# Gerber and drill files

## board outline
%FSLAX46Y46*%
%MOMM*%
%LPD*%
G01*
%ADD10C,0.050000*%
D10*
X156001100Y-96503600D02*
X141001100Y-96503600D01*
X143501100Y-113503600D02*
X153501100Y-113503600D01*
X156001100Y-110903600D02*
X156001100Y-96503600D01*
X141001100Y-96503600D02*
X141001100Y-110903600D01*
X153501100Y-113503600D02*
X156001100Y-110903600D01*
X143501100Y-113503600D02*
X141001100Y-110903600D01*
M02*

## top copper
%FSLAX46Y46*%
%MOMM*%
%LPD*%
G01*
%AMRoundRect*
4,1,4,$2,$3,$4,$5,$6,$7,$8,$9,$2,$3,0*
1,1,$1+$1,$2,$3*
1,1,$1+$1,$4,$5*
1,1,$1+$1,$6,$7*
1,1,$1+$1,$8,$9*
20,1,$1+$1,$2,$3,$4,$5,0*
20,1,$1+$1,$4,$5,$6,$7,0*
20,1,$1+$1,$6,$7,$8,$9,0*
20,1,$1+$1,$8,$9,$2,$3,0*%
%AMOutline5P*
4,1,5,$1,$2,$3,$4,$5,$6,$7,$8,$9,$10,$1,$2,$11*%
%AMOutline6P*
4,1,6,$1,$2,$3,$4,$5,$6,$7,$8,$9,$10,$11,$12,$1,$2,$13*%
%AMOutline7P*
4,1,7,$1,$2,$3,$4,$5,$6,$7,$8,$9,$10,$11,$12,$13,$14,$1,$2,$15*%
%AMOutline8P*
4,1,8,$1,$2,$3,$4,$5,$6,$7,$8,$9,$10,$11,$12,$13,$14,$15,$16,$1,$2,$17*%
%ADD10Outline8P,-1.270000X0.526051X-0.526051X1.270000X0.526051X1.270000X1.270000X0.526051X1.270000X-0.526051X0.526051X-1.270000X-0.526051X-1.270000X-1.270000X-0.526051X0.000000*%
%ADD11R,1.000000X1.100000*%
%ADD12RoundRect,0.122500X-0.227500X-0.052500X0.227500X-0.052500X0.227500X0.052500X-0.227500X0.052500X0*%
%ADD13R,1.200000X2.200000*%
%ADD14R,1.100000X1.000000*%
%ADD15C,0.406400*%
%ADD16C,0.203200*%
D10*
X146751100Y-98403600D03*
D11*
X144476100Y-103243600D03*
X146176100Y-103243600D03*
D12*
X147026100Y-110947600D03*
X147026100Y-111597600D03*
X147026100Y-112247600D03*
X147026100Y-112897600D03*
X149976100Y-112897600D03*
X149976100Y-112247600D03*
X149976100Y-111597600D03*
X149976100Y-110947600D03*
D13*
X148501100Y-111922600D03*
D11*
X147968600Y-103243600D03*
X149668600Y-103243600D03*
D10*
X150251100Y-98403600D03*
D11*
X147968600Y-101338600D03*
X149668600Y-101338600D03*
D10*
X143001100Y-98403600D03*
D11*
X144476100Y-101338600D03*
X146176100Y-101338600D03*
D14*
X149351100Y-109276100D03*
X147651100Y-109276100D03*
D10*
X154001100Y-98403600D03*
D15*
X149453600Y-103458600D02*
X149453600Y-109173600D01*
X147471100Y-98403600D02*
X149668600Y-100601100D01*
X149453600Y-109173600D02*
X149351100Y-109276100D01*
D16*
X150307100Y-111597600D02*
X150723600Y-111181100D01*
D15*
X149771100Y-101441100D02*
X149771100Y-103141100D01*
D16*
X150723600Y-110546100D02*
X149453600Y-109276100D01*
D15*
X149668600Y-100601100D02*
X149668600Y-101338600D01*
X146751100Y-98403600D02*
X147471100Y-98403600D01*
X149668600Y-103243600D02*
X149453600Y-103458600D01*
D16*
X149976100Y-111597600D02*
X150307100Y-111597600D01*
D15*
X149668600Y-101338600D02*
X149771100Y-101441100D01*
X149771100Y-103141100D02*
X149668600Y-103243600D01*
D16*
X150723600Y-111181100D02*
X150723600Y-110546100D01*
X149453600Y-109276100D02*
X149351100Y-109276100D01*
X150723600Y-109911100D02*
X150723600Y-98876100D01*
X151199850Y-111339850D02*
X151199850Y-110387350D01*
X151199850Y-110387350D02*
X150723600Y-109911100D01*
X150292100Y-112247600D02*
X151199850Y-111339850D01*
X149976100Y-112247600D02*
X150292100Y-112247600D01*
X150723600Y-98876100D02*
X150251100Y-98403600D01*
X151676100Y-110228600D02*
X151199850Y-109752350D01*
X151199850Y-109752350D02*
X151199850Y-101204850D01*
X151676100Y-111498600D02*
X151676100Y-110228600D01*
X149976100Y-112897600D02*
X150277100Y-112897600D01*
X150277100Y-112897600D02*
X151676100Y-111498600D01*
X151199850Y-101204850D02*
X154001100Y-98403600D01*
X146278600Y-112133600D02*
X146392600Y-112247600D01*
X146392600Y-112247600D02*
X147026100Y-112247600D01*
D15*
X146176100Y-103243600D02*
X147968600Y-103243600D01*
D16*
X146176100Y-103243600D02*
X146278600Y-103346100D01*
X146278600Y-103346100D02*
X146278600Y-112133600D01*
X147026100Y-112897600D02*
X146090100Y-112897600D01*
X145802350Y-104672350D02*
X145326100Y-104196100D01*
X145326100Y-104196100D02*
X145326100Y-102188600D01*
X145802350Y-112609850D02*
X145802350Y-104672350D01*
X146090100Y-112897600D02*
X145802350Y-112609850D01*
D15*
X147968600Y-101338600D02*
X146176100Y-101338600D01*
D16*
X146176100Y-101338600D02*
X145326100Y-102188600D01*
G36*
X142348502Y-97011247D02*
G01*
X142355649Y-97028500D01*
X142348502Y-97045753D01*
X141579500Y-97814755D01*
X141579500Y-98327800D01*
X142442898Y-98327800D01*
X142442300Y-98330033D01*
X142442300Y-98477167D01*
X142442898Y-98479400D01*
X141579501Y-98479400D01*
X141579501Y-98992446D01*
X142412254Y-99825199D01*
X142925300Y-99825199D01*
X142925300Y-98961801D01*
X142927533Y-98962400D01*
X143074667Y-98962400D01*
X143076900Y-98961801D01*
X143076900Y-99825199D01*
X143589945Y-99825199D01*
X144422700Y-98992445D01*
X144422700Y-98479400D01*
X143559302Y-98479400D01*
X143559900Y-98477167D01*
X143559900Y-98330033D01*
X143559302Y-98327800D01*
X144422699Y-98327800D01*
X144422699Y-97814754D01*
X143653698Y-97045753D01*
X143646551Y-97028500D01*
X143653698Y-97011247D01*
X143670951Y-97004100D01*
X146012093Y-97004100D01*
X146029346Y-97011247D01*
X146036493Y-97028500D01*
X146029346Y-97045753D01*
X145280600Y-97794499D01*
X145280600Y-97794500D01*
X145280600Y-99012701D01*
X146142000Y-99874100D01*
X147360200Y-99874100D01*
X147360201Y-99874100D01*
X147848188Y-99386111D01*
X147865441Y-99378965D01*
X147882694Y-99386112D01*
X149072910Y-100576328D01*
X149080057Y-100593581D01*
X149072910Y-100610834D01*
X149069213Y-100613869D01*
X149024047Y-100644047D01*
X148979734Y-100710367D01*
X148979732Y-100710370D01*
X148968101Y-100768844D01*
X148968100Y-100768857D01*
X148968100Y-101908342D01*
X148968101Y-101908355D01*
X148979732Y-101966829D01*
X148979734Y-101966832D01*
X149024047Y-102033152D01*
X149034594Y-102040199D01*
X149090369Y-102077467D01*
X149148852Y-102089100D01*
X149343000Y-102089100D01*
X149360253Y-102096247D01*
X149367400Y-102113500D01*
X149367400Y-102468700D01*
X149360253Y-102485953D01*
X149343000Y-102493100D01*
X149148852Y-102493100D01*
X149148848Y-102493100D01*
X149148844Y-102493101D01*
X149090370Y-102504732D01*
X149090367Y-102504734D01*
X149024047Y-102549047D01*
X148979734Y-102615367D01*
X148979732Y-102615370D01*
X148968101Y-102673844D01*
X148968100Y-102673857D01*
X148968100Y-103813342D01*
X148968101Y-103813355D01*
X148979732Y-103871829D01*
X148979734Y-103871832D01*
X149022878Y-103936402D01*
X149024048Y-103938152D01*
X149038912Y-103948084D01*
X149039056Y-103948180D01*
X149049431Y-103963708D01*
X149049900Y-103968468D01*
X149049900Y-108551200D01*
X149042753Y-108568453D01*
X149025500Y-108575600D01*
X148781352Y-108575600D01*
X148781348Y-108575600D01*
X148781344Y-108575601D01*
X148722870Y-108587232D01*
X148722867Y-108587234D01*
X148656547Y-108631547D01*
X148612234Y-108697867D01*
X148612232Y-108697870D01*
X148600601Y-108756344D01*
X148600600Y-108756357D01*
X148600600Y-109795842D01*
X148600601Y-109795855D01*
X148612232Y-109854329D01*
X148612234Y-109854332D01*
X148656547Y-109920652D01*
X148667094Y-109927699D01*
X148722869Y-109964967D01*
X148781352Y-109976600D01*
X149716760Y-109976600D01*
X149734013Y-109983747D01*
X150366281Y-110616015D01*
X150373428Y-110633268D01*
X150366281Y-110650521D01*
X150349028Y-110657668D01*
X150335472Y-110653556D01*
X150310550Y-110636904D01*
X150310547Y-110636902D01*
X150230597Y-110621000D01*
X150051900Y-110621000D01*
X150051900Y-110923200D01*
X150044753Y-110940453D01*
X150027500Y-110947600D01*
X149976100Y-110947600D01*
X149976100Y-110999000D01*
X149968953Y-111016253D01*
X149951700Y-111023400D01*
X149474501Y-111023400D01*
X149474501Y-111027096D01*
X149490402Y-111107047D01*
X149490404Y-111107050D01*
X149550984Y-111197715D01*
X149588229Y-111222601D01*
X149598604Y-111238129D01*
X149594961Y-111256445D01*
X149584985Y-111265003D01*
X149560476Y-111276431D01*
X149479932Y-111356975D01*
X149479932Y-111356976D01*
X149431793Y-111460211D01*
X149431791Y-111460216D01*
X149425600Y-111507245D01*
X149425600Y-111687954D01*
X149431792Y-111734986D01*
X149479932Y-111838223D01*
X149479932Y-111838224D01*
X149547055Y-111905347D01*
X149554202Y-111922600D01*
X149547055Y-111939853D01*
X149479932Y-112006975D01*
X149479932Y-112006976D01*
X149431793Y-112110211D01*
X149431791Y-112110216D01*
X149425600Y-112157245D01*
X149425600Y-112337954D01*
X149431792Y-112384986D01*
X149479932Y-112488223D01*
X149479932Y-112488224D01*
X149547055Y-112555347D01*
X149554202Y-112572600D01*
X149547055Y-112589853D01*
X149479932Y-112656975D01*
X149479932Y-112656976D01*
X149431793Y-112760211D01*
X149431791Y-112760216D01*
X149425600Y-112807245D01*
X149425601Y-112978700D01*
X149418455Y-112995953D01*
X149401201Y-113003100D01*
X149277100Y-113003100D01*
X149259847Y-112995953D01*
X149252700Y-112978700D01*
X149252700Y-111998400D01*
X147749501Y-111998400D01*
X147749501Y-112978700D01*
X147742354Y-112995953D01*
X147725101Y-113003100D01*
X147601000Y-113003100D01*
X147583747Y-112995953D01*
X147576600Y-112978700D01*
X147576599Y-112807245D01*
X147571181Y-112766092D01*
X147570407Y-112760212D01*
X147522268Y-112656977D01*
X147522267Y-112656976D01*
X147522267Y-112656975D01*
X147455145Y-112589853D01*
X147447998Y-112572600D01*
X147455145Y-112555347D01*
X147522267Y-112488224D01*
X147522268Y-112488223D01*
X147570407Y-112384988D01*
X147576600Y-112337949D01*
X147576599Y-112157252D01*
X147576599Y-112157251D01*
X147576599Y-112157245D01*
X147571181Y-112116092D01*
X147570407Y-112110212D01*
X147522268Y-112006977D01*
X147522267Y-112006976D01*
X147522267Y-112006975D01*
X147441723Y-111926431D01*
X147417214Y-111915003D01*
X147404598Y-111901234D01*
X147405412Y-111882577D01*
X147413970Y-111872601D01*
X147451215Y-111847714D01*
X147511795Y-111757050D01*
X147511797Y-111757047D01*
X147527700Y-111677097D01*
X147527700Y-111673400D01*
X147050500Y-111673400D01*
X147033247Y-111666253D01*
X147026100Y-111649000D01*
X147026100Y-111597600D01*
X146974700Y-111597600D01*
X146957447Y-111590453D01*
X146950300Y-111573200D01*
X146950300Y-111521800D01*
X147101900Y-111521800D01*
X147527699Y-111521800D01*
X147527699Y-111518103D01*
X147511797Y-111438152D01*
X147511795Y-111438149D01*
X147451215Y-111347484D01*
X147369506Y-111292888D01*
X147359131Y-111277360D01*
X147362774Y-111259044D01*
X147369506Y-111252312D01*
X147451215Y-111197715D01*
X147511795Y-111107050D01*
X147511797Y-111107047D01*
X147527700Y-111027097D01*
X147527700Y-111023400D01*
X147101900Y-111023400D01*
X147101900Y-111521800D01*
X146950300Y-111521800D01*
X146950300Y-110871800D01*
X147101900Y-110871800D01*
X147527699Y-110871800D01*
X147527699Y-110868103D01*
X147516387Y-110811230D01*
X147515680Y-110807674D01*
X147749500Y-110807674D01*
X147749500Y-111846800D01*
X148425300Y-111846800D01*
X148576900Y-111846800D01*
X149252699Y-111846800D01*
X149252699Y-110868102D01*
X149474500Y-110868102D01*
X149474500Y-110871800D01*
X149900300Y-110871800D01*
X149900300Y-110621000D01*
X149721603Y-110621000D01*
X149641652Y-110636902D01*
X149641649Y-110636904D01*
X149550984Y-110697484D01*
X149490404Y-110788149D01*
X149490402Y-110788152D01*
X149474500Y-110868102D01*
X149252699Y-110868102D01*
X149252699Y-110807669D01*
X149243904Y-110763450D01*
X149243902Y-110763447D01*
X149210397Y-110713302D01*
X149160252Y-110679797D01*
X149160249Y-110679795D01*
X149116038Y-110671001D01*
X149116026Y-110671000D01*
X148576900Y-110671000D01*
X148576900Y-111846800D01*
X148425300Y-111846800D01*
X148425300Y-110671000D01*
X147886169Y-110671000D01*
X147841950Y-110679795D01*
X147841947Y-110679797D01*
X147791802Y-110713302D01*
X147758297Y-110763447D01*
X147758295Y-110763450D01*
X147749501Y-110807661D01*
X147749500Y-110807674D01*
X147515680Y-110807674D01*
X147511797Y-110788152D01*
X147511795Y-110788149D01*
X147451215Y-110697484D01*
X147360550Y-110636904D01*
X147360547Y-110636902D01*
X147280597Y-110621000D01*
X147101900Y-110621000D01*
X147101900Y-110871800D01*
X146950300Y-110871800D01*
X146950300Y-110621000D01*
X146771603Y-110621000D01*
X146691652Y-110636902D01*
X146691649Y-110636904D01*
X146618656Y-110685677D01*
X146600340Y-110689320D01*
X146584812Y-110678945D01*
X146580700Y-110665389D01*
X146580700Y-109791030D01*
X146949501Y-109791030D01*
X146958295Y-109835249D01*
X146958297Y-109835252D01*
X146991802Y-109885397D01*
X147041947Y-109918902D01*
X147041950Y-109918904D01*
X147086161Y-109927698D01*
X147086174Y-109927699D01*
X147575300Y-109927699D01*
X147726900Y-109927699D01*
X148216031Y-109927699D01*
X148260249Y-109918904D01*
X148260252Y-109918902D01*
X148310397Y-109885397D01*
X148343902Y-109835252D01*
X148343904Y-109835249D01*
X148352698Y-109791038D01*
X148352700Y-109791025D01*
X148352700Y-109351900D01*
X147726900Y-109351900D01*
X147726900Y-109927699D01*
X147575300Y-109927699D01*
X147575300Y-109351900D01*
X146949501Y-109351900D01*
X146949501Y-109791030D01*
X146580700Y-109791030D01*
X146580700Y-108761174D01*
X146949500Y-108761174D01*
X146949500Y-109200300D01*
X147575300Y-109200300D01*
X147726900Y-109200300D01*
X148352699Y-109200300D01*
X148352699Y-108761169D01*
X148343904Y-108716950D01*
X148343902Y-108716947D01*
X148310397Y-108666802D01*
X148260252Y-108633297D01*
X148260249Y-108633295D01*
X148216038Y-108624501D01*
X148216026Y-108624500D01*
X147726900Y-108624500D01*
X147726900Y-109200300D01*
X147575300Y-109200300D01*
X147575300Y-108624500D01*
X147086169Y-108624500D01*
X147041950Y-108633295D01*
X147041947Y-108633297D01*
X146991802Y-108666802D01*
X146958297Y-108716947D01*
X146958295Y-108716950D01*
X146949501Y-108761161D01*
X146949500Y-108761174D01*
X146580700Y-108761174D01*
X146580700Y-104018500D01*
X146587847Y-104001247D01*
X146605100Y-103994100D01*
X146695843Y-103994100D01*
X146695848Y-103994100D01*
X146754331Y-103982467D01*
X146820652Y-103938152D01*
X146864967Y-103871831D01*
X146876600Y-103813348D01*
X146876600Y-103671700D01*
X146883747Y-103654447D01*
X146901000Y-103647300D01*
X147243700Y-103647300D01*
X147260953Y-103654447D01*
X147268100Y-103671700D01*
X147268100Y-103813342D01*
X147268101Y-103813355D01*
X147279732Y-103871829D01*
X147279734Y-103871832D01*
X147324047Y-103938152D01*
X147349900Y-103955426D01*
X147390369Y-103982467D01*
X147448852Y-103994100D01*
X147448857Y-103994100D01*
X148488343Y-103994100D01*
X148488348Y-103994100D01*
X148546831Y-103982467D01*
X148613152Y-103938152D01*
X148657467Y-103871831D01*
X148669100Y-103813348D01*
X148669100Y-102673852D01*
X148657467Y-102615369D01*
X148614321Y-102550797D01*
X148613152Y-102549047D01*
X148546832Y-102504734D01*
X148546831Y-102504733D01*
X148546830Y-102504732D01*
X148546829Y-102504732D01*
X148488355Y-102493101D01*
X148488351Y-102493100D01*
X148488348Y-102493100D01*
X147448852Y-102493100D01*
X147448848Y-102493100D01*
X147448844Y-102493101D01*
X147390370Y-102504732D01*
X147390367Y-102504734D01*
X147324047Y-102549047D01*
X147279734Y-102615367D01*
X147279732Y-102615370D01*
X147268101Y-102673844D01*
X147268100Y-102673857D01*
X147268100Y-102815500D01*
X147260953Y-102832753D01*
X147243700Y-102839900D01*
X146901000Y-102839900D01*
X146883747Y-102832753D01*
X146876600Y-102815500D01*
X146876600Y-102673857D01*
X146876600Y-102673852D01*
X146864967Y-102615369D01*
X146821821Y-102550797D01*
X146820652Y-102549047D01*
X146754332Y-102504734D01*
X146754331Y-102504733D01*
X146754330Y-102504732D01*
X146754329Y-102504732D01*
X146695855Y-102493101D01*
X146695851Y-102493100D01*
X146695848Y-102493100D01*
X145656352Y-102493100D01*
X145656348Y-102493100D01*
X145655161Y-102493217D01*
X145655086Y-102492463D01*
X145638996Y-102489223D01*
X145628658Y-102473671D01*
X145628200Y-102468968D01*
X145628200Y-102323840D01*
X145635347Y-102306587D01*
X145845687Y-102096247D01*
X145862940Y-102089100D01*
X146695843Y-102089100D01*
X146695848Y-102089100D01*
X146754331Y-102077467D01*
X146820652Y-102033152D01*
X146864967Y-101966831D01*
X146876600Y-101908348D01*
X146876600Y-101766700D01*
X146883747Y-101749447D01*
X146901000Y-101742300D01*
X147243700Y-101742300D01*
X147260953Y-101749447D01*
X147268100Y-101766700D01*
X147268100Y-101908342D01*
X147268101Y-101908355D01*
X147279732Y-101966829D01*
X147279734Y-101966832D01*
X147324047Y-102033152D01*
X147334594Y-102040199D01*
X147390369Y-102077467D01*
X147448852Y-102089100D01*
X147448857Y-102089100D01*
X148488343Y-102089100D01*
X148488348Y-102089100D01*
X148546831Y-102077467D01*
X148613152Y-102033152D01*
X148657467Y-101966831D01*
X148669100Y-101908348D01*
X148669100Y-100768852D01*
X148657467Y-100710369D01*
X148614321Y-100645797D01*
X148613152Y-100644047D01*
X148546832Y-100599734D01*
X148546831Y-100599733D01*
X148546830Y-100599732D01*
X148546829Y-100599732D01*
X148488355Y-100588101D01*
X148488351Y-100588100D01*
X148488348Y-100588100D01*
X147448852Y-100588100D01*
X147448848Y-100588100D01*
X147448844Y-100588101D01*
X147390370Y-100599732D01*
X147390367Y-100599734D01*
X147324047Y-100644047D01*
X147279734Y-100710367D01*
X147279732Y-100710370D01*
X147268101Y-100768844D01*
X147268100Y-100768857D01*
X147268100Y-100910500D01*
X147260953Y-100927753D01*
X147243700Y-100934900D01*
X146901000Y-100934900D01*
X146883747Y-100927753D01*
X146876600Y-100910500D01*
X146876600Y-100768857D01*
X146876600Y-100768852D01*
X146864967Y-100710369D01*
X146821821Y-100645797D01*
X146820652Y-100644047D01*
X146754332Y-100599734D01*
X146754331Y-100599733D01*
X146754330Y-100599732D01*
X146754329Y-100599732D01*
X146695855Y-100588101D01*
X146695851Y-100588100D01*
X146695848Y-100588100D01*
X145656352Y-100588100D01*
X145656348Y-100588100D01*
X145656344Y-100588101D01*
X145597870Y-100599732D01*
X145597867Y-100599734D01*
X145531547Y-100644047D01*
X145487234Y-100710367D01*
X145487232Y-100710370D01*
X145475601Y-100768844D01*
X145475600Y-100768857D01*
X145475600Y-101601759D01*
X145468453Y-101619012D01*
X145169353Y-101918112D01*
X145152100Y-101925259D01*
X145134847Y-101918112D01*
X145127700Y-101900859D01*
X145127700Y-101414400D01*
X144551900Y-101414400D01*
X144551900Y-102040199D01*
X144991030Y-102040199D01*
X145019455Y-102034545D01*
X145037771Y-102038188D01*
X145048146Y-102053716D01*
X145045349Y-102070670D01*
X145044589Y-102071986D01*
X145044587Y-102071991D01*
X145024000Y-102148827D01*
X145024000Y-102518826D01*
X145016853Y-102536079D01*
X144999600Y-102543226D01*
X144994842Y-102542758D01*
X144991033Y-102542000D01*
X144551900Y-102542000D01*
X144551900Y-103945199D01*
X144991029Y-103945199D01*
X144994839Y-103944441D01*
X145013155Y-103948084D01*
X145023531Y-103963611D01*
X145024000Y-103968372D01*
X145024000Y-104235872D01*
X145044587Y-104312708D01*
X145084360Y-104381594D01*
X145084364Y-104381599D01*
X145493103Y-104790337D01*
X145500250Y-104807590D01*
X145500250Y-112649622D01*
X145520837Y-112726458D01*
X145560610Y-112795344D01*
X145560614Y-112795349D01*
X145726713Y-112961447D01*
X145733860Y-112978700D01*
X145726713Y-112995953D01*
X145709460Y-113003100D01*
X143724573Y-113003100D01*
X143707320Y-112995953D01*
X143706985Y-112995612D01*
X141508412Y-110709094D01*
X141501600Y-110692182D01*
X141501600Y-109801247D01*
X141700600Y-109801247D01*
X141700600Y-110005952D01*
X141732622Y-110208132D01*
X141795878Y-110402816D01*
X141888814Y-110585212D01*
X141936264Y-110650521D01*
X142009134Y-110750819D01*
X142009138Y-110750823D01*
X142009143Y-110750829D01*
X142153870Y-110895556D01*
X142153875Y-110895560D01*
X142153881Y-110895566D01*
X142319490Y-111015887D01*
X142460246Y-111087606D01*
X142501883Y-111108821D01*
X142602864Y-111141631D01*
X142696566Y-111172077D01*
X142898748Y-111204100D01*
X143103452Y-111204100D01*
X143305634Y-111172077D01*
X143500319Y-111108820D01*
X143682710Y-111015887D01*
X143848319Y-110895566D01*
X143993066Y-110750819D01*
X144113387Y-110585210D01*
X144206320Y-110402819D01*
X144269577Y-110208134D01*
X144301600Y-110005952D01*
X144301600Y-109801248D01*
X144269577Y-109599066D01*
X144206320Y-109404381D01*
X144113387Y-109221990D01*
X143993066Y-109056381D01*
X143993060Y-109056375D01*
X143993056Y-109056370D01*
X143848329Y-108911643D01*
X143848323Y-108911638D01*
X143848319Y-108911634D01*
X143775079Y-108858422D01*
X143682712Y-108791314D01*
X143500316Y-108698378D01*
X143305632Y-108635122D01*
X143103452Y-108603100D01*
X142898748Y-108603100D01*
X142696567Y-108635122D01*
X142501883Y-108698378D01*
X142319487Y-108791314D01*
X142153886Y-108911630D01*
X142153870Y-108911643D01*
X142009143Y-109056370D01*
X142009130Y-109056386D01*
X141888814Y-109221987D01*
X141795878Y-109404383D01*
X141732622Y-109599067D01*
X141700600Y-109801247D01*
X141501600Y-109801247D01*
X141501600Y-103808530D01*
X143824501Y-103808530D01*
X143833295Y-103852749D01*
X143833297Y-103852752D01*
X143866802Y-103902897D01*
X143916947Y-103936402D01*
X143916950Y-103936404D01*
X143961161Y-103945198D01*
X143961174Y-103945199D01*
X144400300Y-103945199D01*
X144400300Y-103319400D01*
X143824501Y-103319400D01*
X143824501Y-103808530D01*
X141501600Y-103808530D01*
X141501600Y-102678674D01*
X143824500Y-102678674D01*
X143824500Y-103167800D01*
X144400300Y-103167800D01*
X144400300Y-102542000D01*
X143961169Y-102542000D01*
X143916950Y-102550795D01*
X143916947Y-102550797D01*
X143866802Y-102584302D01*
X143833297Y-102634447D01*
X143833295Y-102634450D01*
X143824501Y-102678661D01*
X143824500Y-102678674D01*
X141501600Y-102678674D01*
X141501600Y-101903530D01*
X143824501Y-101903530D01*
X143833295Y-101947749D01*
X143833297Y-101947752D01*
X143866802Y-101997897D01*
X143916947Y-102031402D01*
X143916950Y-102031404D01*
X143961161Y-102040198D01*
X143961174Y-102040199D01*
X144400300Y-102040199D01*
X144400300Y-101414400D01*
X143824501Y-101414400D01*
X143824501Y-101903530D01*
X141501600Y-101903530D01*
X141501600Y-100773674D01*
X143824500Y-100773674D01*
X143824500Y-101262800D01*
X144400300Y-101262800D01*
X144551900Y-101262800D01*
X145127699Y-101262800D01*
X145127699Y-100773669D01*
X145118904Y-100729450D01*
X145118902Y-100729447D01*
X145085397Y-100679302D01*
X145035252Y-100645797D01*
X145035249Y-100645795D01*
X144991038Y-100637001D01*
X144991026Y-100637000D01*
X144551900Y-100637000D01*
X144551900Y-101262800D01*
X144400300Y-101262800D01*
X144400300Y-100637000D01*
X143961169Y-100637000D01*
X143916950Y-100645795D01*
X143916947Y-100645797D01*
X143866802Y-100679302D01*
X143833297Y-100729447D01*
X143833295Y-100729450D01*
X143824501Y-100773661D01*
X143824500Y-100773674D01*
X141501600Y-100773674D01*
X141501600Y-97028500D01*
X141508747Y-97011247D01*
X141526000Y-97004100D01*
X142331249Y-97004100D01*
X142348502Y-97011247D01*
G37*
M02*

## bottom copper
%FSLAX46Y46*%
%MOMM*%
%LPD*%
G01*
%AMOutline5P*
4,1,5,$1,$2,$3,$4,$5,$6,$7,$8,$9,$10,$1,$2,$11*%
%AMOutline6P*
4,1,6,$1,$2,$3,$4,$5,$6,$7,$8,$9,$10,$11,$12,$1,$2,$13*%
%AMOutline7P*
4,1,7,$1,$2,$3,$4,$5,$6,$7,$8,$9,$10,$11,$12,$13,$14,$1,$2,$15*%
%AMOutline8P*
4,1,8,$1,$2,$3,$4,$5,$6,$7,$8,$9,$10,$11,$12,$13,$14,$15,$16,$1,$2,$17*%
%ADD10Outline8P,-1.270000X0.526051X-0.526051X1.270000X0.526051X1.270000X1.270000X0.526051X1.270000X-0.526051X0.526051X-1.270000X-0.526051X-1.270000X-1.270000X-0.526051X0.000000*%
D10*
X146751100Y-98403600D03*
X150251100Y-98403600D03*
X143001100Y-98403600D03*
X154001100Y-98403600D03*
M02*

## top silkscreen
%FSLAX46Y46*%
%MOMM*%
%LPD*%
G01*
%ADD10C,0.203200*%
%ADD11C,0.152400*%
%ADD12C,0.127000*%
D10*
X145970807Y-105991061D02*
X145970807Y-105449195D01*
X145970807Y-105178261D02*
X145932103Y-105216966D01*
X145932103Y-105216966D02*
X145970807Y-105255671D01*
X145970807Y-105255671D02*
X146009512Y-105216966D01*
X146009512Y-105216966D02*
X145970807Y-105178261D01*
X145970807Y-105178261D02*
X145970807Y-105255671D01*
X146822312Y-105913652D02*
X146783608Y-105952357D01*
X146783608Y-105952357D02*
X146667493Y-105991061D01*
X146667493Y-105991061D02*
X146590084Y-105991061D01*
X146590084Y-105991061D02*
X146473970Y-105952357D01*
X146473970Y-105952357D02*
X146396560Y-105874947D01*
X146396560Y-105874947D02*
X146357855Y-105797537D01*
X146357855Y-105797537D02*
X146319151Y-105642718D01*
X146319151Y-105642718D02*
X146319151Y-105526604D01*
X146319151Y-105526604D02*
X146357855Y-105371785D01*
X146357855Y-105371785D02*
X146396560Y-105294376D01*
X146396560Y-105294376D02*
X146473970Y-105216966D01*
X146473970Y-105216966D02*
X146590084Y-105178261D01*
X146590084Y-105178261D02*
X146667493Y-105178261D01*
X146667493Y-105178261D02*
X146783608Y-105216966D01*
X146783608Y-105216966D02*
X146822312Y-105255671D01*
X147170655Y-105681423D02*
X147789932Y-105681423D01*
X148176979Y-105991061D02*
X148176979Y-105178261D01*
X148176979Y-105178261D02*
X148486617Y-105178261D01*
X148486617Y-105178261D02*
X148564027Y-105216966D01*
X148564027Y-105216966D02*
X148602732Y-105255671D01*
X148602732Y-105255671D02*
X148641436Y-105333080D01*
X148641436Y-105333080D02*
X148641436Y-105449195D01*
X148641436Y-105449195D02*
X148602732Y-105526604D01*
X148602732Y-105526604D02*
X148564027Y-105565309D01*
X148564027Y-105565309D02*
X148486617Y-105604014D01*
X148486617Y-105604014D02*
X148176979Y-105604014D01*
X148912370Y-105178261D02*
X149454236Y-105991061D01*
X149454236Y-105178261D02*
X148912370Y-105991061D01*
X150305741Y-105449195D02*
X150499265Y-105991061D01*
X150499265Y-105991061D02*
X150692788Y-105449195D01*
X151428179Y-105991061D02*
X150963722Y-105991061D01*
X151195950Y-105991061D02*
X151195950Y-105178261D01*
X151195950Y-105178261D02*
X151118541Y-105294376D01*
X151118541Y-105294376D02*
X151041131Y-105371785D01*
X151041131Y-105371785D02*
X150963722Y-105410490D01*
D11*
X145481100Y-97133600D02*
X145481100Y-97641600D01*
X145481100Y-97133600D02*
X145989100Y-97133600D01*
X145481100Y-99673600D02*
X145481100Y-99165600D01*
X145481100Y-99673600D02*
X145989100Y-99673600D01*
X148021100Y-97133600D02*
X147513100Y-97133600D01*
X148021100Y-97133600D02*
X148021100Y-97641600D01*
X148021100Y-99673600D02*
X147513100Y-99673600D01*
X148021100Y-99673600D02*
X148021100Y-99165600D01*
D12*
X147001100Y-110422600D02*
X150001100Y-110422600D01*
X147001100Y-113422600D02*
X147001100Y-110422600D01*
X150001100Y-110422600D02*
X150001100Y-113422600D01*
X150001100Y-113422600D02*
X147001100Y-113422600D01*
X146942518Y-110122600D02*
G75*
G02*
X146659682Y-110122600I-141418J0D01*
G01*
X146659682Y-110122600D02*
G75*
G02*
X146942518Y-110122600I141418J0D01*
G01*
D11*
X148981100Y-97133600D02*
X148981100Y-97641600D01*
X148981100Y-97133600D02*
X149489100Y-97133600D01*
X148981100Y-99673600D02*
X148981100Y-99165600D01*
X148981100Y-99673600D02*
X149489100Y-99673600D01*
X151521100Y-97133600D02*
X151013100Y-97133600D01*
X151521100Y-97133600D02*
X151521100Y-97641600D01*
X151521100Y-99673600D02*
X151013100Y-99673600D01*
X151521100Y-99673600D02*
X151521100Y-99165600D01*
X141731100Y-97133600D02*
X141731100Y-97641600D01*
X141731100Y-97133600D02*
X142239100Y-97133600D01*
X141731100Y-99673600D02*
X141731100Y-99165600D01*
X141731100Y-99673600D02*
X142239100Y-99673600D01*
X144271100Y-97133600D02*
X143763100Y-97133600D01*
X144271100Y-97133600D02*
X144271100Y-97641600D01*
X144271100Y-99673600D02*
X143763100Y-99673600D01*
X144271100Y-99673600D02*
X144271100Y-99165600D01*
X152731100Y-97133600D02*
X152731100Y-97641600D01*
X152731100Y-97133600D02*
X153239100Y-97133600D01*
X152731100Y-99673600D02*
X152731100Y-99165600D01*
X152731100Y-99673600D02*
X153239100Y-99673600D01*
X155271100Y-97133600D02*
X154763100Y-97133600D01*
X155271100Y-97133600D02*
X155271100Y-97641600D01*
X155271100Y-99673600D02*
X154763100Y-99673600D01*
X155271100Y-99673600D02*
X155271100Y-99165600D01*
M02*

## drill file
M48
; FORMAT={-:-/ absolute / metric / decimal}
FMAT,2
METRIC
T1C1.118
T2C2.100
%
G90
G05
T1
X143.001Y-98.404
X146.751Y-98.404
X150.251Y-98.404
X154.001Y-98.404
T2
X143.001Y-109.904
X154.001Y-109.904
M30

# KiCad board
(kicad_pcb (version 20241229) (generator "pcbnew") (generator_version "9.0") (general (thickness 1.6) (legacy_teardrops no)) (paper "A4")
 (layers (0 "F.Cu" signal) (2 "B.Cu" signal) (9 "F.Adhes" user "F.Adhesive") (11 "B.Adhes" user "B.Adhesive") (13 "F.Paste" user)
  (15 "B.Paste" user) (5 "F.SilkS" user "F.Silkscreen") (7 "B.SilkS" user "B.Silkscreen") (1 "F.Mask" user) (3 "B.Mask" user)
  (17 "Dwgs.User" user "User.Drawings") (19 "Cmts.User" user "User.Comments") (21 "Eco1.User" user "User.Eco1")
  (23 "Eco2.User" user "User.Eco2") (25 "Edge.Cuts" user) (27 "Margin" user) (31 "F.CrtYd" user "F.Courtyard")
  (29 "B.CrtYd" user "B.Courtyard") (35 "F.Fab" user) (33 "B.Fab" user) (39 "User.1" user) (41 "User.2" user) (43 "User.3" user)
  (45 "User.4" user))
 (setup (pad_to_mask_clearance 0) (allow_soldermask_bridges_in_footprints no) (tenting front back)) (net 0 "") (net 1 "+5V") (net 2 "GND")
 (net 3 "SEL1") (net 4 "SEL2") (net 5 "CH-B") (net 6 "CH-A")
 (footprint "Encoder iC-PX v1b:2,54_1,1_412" (layer "F.Cu") (at 146.7511 98.4036)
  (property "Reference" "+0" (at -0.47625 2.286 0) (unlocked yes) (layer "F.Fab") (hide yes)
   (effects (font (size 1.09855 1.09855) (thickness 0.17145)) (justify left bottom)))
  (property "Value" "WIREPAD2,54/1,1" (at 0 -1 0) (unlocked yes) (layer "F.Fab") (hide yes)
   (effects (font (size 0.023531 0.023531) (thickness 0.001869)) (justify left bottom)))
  (fp_line (start -1.27 -1.27) (end -1.27 -0.762) (stroke (width 0.1524) (type solid)) (layer "F.SilkS"))
  (fp_line (start -1.27 -1.27) (end -0.762 -1.27) (stroke (width 0.1524) (type solid)) (layer "F.SilkS"))
  (fp_line (start -1.27 1.27) (end -1.27 0.762) (stroke (width 0.1524) (type solid)) (layer "F.SilkS"))
  (fp_line (start -1.27 1.27) (end -0.762 1.27) (stroke (width 0.1524) (type solid)) (layer "F.SilkS"))
  (fp_line (start 1.27 -1.27) (end 0.762 -1.27) (stroke (width 0.1524) (type solid)) (layer "F.SilkS"))
  (fp_line (start 1.27 -1.27) (end 1.27 -0.762) (stroke (width 0.1524) (type solid)) (layer "F.SilkS"))
  (fp_line (start 1.27 1.27) (end 0.762 1.27) (stroke (width 0.1524) (type solid)) (layer "F.SilkS"))
  (fp_line (start 1.27 1.27) (end 1.27 0.762) (stroke (width 0.1524) (type solid)) (layer "F.SilkS"))
  (pad "1" thru_hole roundrect (at 0 0) (size 2.54 2.54) (drill 1.1176) (layers "*.Cu" "*.Mask") (remove_unused_layers no)
   (roundrect_rratio 0.25) (chamfer_ratio 0.2928932188) (chamfer top_left top_right bottom_left bottom_right) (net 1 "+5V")
   (solder_mask_margin 0.075) (thermal_bridge_angle 0)))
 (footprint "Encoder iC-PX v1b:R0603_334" (layer "F.Cu") (at 145.3261 103.2436)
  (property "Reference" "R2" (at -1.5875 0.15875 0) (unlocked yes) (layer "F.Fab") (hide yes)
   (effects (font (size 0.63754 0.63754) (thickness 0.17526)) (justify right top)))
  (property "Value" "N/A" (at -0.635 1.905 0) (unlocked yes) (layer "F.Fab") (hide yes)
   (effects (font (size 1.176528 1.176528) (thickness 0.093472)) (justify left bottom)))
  (pad "1" smd rect (at -0.85 0) (size 1 1.1) (layers "F.Cu" "F.Mask" "F.Paste") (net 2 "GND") (solder_mask_margin 0.075)
   (solder_paste_margin 0) (thermal_bridge_angle 0))
  (pad "2" smd rect (at 0.85 0) (size 1 1.1) (layers "F.Cu" "F.Mask" "F.Paste") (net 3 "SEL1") (solder_mask_margin 0.075)
   (solder_paste_margin 0) (thermal_bridge_angle 0)))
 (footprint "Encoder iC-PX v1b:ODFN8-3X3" (layer "F.Cu") (at 148.5011 111.9226)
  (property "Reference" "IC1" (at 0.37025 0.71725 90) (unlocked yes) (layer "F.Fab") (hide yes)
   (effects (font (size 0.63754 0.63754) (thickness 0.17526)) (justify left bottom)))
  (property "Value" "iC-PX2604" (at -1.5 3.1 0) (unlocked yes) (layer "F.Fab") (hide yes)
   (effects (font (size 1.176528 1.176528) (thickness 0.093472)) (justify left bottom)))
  (fp_line (start -1.5 -1.5) (end 1.5 -1.5) (stroke (width 0.127) (type solid)) (layer "F.SilkS"))
  (fp_line (start -1.5 1.5) (end -1.5 -1.5) (stroke (width 0.127) (type solid)) (layer "F.SilkS"))
  (fp_line (start 1.5 -1.5) (end 1.5 1.5) (stroke (width 0.127) (type solid)) (layer "F.SilkS"))
  (fp_line (start 1.5 1.5) (end -1.5 1.5) (stroke (width 0.127) (type solid)) (layer "F.SilkS"))
  (fp_circle (center -1.7 -1.8) (end -1.558582 -1.8) (stroke (width 0.127) (type solid)) (fill no) (layer "F.SilkS"))
  (pad "1" smd roundrect (at -1.475 -0.975) (size 0.7 0.35) (layers "F.Cu" "F.Mask" "F.Paste") (roundrect_rratio 0.35) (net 2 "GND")
   (solder_mask_margin 0.075) (solder_paste_margin 0) (thermal_bridge_angle 0))
  (pad "2" smd roundrect (at -1.475 -0.325) (size 0.7 0.35) (layers "F.Cu" "F.Mask" "F.Paste") (roundrect_rratio 0.35) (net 2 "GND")
   (solder_mask_margin 0.075) (solder_paste_margin 0) (thermal_bridge_angle 0))
  (pad "3" smd roundrect (at -1.475 0.325) (size 0.7 0.35) (layers "F.Cu" "F.Mask" "F.Paste") (roundrect_rratio 0.35) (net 3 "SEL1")
   (solder_mask_margin 0.075) (solder_paste_margin 0) (thermal_bridge_angle 0))
  (pad "4" smd roundrect (at -1.475 0.975) (size 0.7 0.35) (layers "F.Cu" "F.Mask" "F.Paste") (roundrect_rratio 0.35) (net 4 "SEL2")
   (solder_mask_margin 0.075) (solder_paste_margin 0) (thermal_bridge_angle 0))
  (pad "5" smd roundrect (at 1.475 0.975) (size 0.7 0.35) (layers "F.Cu" "F.Mask" "F.Paste") (roundrect_rratio 0.35) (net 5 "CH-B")
   (solder_mask_margin 0.075) (solder_paste_margin 0) (thermal_bridge_angle 0))
  (pad "6" smd roundrect (at 1.475 0.325) (size 0.7 0.35) (layers "F.Cu" "F.Mask" "F.Paste") (roundrect_rratio 0.35) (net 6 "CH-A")
   (solder_mask_margin 0.075) (solder_paste_margin 0) (thermal_bridge_angle 0))
  (pad "7" smd roundrect (at 1.475 -0.325) (size 0.7 0.35) (layers "F.Cu" "F.Mask" "F.Paste") (roundrect_rratio 0.35) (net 1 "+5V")
   (solder_mask_margin 0.075) (solder_paste_margin 0) (thermal_bridge_angle 0))
  (pad "8" smd roundrect (at 1.475 -0.975) (size 0.7 0.35) (layers "F.Cu" "F.Mask" "F.Paste") (roundrect_rratio 0.35) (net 2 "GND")
   (solder_mask_margin 0.075) (solder_paste_margin 0) (thermal_bridge_angle 0))
  (pad "BP" smd rect (at 0 0) (size 1.2 2.2) (layers "F.Cu" "F.Mask") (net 2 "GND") (solder_mask_margin 0.075) (solder_paste_margin 0)
   (thermal_bridge_angle 0)))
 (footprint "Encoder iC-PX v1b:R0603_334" (layer "F.Cu") (at 148.8186 103.2436)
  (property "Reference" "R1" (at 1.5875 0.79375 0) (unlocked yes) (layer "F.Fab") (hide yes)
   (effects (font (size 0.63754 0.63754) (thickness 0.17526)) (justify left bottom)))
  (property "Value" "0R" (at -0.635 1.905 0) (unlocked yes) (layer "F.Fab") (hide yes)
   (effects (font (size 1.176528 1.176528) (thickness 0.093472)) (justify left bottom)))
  (pad "1" smd rect (at -0.85 0) (size 1 1.1) (layers "F.Cu" "F.Mask" "F.Paste") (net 3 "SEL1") (solder_mask_margin 0.075)
   (solder_paste_margin 0) (thermal_bridge_angle 0))
  (pad "2" smd rect (at 0.85 0) (size 1 1.1) (layers "F.Cu" "F.Mask" "F.Paste") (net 1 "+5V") (solder_mask_margin 0.075)
   (solder_paste_margin 0) (thermal_bridge_angle 0)))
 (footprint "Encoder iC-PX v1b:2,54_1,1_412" (layer "F.Cu") (at 150.2511 98.4036)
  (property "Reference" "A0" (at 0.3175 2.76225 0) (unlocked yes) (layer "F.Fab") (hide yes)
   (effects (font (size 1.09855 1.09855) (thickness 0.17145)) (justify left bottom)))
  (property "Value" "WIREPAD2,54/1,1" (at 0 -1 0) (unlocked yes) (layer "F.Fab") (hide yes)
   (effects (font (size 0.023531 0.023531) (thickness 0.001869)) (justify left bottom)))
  (fp_line (start -1.27 -1.27) (end -1.27 -0.762) (stroke (width 0.1524) (type solid)) (layer "F.SilkS"))
  (fp_line (start -1.27 -1.27) (end -0.762 -1.27) (stroke (width 0.1524) (type solid)) (layer "F.SilkS"))
  (fp_line (start -1.27 1.27) (end -1.27 0.762) (stroke (width 0.1524) (type solid)) (layer "F.SilkS"))
  (fp_line (start -1.27 1.27) (end -0.762 1.27) (stroke (width 0.1524) (type solid)) (layer "F.SilkS"))
  (fp_line (start 1.27 -1.27) (end 0.762 -1.27) (stroke (width 0.1524) (type solid)) (layer "F.SilkS"))
  (fp_line (start 1.27 -1.27) (end 1.27 -0.762) (stroke (width 0.1524) (type solid)) (layer "F.SilkS"))
  (fp_line (start 1.27 1.27) (end 0.762 1.27) (stroke (width 0.1524) (type solid)) (layer "F.SilkS"))
  (fp_line (start 1.27 1.27) (end 1.27 0.762) (stroke (width 0.1524) (type solid)) (layer "F.SilkS"))
  (pad "1" thru_hole roundrect (at 0 0) (size 2.54 2.54) (drill 1.1176) (layers "*.Cu" "*.Mask") (remove_unused_layers no)
   (roundrect_rratio 0.25) (chamfer_ratio 0.2928932188) (chamfer top_left top_right bottom_left bottom_right) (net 6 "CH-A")
   (solder_mask_margin 0.075) (thermal_bridge_angle 0)))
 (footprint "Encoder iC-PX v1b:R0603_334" (layer "F.Cu") (at 148.8186 101.3386)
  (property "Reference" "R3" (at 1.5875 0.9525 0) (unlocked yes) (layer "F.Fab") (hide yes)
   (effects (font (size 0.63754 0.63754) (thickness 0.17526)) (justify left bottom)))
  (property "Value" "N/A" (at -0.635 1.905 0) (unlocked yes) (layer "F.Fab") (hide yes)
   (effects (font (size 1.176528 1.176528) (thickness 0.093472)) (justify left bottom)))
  (pad "1" smd rect (at -0.85 0) (size 1 1.1) (layers "F.Cu" "F.Mask" "F.Paste") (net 4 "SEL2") (solder_mask_margin 0.075)
   (solder_paste_margin 0) (thermal_bridge_angle 0))
  (pad "2" smd rect (at 0.85 0) (size 1 1.1) (layers "F.Cu" "F.Mask" "F.Paste") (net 1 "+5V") (solder_mask_margin 0.075)
   (solder_paste_margin 0) (thermal_bridge_angle 0)))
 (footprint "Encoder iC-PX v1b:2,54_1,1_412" (layer "F.Cu") (at 143.0011 98.4036)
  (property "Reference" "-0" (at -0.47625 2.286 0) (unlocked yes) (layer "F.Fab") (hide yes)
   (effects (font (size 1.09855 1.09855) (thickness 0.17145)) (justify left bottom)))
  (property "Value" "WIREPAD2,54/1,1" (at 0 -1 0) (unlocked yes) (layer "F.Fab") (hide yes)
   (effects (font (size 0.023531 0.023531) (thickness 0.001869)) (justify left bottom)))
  (fp_line (start -1.27 -1.27) (end -1.27 -0.762) (stroke (width 0.1524) (type solid)) (layer "F.SilkS"))
  (fp_line (start -1.27 -1.27) (end -0.762 -1.27) (stroke (width 0.1524) (type solid)) (layer "F.SilkS"))
  (fp_line (start -1.27 1.27) (end -1.27 0.762) (stroke (width 0.1524) (type solid)) (layer "F.SilkS"))
  (fp_line (start -1.27 1.27) (end -0.762 1.27) (stroke (width 0.1524) (type solid)) (layer "F.SilkS"))
  (fp_line (start 1.27 -1.27) (end 0.762 -1.27) (stroke (width 0.1524) (type solid)) (layer "F.SilkS"))
  (fp_line (start 1.27 -1.27) (end 1.27 -0.762) (stroke (width 0.1524) (type solid)) (layer "F.SilkS"))
  (fp_line (start 1.27 1.27) (end 0.762 1.27) (stroke (width 0.1524) (type solid)) (layer "F.SilkS"))
  (fp_line (start 1.27 1.27) (end 1.27 0.762) (stroke (width 0.1524) (type solid)) (layer "F.SilkS"))
  (pad "1" thru_hole roundrect (at 0 0) (size 2.54 2.54) (drill 1.1176) (layers "*.Cu" "*.Mask") (remove_unused_layers no)
   (roundrect_rratio 0.25) (chamfer_ratio 0.2928932188) (chamfer top_left top_right bottom_left bottom_right) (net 2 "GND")
   (solder_mask_margin 0.075) (thermal_bridge_angle 0)))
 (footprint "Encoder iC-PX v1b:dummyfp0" (layer "F.Cu") (at 143.0011 109.9036)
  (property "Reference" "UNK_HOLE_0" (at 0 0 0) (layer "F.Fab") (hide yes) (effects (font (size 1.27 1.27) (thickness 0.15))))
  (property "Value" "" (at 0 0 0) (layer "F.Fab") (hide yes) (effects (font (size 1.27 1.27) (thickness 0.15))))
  (pad "" np_thru_hole circle (at 0 0) (size 2.1 2.1) (drill 2.1) (layers "*.Cu" "*.Mask")))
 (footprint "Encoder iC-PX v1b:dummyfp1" (layer "F.Cu") (at 154.0011 109.9036)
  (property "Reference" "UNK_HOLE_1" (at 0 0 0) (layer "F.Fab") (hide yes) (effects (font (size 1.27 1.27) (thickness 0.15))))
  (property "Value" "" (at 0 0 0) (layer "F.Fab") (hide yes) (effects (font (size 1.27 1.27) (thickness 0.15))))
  (pad "" np_thru_hole circle (at 0 0) (size 2.1 2.1) (drill 2.1) (layers "*.Cu" "*.Mask")))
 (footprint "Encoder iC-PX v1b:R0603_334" (layer "F.Cu") (at 145.3261 101.3386)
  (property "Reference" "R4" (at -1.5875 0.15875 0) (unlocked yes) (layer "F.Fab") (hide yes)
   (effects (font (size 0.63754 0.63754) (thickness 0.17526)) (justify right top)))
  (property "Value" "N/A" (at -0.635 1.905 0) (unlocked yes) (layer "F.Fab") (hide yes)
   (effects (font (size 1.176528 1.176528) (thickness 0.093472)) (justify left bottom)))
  (pad "1" smd rect (at -0.85 0) (size 1 1.1) (layers "F.Cu" "F.Mask" "F.Paste") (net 2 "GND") (solder_mask_margin 0.075)
   (solder_paste_margin 0) (thermal_bridge_angle 0))
  (pad "2" smd rect (at 0.85 0) (size 1 1.1) (layers "F.Cu" "F.Mask" "F.Paste") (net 4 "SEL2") (solder_mask_margin 0.075)
   (solder_paste_margin 0) (thermal_bridge_angle 0)))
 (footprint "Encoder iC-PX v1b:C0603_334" (layer "F.Cu") (at 148.5011 109.2761 180)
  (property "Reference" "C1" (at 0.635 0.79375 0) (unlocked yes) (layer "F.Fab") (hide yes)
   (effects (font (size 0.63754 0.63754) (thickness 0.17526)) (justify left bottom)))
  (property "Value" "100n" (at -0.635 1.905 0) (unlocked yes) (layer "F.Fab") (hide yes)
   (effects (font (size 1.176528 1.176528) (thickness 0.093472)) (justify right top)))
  (pad "1" smd rect (at -0.85 0 180) (size 1.1 1) (layers "F.Cu" "F.Mask" "F.Paste") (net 1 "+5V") (solder_mask_margin 0.075)
   (solder_paste_margin 0) (thermal_bridge_angle 0))
  (pad "2" smd rect (at 0.85 0 180) (size 1.1 1) (layers "F.Cu" "F.Mask" "F.Paste") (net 2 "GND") (solder_mask_margin 0.075)
   (solder_paste_margin 0) (thermal_bridge_angle 0)))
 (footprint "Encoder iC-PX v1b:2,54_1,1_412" (layer "F.Cu") (at 154.0011 98.4036)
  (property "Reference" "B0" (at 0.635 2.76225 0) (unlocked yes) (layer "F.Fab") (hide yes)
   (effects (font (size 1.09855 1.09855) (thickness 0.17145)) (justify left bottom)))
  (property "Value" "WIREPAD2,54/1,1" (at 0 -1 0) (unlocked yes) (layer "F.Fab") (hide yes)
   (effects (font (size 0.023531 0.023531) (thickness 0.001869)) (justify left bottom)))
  (fp_line (start -1.27 -1.27) (end -1.27 -0.762) (stroke (width 0.1524) (type solid)) (layer "F.SilkS"))
  (fp_line (start -1.27 -1.27) (end -0.762 -1.27) (stroke (width 0.1524) (type solid)) (layer "F.SilkS"))
  (fp_line (start -1.27 1.27) (end -1.27 0.762) (stroke (width 0.1524) (type solid)) (layer "F.SilkS"))
  (fp_line (start -1.27 1.27) (end -0.762 1.27) (stroke (width 0.1524) (type solid)) (layer "F.SilkS"))
  (fp_line (start 1.27 -1.27) (end 0.762 -1.27) (stroke (width 0.1524) (type solid)) (layer "F.SilkS"))
  (fp_line (start 1.27 -1.27) (end 1.27 -0.762) (stroke (width 0.1524) (type solid)) (layer "F.SilkS"))
  (fp_line (start 1.27 1.27) (end 0.762 1.27) (stroke (width 0.1524) (type solid)) (layer "F.SilkS"))
  (fp_line (start 1.27 1.27) (end 1.27 0.762) (stroke (width 0.1524) (type solid)) (layer "F.SilkS"))
  (pad "1" thru_hole roundrect (at 0 0) (size 2.54 2.54) (drill 1.1176) (layers "*.Cu" "*.Mask") (remove_unused_layers no)
   (roundrect_rratio 0.25) (chamfer_ratio 0.2928932188) (chamfer top_left top_right bottom_left bottom_right) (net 5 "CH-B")
   (solder_mask_margin 0.075) (thermal_bridge_angle 0)))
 (gr_line (start 156.0011 96.5036) (end 141.0011 96.5036) (stroke (width 0.05) (type solid)) (layer "Edge.Cuts"))
 (gr_line (start 143.5011 113.5036) (end 153.5011 113.5036) (stroke (width 0.05) (type solid)) (layer "Edge.Cuts"))
 (gr_line (start 156.0011 110.9036) (end 156.0011 96.5036) (stroke (width 0.05) (type solid)) (layer "Edge.Cuts"))
 (gr_line (start 141.0011 96.5036) (end 141.0011 110.9036) (stroke (width 0.05) (type solid)) (layer "Edge.Cuts"))
 (gr_line (start 153.5011 113.5036) (end 156.0011 110.9036) (stroke (width 0.05) (type solid)) (layer "Edge.Cuts"))
 (gr_line (start 143.5011 113.5036) (end 141.0011 110.9036) (stroke (width 0.05) (type solid)) (layer "Edge.Cuts"))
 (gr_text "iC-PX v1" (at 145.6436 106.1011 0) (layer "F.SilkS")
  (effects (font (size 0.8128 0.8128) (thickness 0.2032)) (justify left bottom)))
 (segment (start 149.4536 103.4586) (end 149.4536 109.1736) (width 0.4064) (layer "F.Cu") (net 1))
 (segment (start 147.4711 98.4036) (end 149.6686 100.6011) (width 0.4064) (layer "F.Cu") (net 1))
 (segment (start 149.4536 109.1736) (end 149.3511 109.2761) (width 0.4064) (layer "F.Cu") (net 1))
 (segment (start 150.3071 111.5976) (end 150.7236 111.1811) (width 0.2032) (layer "F.Cu") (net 1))
 (segment (start 149.7711 101.4411) (end 149.7711 103.1411) (width 0.4064) (layer "F.Cu") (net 1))
 (segment (start 150.7236 110.5461) (end 149.4536 109.2761) (width 0.2032) (layer "F.Cu") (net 1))
 (segment (start 149.6686 100.6011) (end 149.6686 101.3386) (width 0.4064) (layer "F.Cu") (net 1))
 (segment (start 146.7511 98.4036) (end 147.4711 98.4036) (width 0.4064) (layer "F.Cu") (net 1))
 (segment (start 149.6686 103.2436) (end 149.4536 103.4586) (width 0.4064) (layer "F.Cu") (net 1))
 (segment (start 149.9761 111.5976) (end 150.3071 111.5976) (width 0.2032) (layer "F.Cu") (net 1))
 (segment (start 149.6686 101.3386) (end 149.7711 101.4411) (width 0.4064) (layer "F.Cu") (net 1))
 (segment (start 149.7711 103.1411) (end 149.6686 103.2436) (width 0.4064) (layer "F.Cu") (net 1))
 (segment (start 150.7236 111.1811) (end 150.7236 110.5461) (width 0.2032) (layer "F.Cu") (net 1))
 (segment (start 149.4536 109.2761) (end 149.3511 109.2761) (width 0.2032) (layer "F.Cu") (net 1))
 (segment (start 150.7236 109.9111) (end 150.7236 98.8761) (width 0.2032) (layer "F.Cu") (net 6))
 (segment (start 151.19985 111.33985) (end 151.19985 110.38735) (width 0.2032) (layer "F.Cu") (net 6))
 (segment (start 151.19985 110.38735) (end 150.7236 109.9111) (width 0.2032) (layer "F.Cu") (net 6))
 (segment (start 150.2921 112.2476) (end 151.19985 111.33985) (width 0.2032) (layer "F.Cu") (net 6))
 (segment (start 149.9761 112.2476) (end 150.2921 112.2476) (width 0.2032) (layer "F.Cu") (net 6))
 (segment (start 150.7236 98.8761) (end 150.2511 98.4036) (width 0.2032) (layer "F.Cu") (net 6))
 (segment (start 151.6761 110.2286) (end 151.19985 109.75235) (width 0.2032) (layer "F.Cu") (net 5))
 (segment (start 151.19985 109.75235) (end 151.19985 101.20485) (width 0.2032) (layer "F.Cu") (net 5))
 (segment (start 151.6761 111.4986) (end 151.6761 110.2286) (width 0.2032) (layer "F.Cu") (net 5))
 (segment (start 149.9761 112.8976) (end 150.2771 112.8976) (width 0.2032) (layer "F.Cu") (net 5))
 (segment (start 150.2771 112.8976) (end 151.6761 111.4986) (width 0.2032) (layer "F.Cu") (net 5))
 (segment (start 151.19985 101.20485) (end 154.0011 98.4036) (width 0.2032) (layer "F.Cu") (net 5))
 (segment (start 146.2786 112.1336) (end 146.3926 112.2476) (width 0.2032) (layer "F.Cu") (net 3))
 (segment (start 146.3926 112.2476) (end 147.0261 112.2476) (width 0.2032) (layer "F.Cu") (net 3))
 (segment (start 146.1761 103.2436) (end 147.9686 103.2436) (width 0.4064) (layer "F.Cu") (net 3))
 (segment (start 146.1761 103.2436) (end 146.2786 103.3461) (width 0.2032) (layer "F.Cu") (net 3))
 (segment (start 146.2786 103.3461) (end 146.2786 112.1336) (width 0.2032) (layer "F.Cu") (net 3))
 (segment (start 147.0261 112.8976) (end 146.0901 112.8976) (width 0.2032) (layer "F.Cu") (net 4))
 (segment (start 145.80235 104.67235) (end 145.3261 104.1961) (width 0.2032) (layer "F.Cu") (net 4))
 (segment (start 145.3261 104.1961) (end 145.3261 102.1886) (width 0.2032) (layer "F.Cu") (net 4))
 (segment (start 145.80235 112.60985) (end 145.80235 104.67235) (width 0.2032) (layer "F.Cu") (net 4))
 (segment (start 146.0901 112.8976) (end 145.80235 112.60985) (width 0.2032) (layer "F.Cu") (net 4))
 (segment (start 147.9686 101.3386) (end 146.1761 101.3386) (width 0.4064) (layer "F.Cu") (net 4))
 (segment (start 146.1761 101.3386) (end 145.3261 102.1886) (width 0.2032) (layer "F.Cu") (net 4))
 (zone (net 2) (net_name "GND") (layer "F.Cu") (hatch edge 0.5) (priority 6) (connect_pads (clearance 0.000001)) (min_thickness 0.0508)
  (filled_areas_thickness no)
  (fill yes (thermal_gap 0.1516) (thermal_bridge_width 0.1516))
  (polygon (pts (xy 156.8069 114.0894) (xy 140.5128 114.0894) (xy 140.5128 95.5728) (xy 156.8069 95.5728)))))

